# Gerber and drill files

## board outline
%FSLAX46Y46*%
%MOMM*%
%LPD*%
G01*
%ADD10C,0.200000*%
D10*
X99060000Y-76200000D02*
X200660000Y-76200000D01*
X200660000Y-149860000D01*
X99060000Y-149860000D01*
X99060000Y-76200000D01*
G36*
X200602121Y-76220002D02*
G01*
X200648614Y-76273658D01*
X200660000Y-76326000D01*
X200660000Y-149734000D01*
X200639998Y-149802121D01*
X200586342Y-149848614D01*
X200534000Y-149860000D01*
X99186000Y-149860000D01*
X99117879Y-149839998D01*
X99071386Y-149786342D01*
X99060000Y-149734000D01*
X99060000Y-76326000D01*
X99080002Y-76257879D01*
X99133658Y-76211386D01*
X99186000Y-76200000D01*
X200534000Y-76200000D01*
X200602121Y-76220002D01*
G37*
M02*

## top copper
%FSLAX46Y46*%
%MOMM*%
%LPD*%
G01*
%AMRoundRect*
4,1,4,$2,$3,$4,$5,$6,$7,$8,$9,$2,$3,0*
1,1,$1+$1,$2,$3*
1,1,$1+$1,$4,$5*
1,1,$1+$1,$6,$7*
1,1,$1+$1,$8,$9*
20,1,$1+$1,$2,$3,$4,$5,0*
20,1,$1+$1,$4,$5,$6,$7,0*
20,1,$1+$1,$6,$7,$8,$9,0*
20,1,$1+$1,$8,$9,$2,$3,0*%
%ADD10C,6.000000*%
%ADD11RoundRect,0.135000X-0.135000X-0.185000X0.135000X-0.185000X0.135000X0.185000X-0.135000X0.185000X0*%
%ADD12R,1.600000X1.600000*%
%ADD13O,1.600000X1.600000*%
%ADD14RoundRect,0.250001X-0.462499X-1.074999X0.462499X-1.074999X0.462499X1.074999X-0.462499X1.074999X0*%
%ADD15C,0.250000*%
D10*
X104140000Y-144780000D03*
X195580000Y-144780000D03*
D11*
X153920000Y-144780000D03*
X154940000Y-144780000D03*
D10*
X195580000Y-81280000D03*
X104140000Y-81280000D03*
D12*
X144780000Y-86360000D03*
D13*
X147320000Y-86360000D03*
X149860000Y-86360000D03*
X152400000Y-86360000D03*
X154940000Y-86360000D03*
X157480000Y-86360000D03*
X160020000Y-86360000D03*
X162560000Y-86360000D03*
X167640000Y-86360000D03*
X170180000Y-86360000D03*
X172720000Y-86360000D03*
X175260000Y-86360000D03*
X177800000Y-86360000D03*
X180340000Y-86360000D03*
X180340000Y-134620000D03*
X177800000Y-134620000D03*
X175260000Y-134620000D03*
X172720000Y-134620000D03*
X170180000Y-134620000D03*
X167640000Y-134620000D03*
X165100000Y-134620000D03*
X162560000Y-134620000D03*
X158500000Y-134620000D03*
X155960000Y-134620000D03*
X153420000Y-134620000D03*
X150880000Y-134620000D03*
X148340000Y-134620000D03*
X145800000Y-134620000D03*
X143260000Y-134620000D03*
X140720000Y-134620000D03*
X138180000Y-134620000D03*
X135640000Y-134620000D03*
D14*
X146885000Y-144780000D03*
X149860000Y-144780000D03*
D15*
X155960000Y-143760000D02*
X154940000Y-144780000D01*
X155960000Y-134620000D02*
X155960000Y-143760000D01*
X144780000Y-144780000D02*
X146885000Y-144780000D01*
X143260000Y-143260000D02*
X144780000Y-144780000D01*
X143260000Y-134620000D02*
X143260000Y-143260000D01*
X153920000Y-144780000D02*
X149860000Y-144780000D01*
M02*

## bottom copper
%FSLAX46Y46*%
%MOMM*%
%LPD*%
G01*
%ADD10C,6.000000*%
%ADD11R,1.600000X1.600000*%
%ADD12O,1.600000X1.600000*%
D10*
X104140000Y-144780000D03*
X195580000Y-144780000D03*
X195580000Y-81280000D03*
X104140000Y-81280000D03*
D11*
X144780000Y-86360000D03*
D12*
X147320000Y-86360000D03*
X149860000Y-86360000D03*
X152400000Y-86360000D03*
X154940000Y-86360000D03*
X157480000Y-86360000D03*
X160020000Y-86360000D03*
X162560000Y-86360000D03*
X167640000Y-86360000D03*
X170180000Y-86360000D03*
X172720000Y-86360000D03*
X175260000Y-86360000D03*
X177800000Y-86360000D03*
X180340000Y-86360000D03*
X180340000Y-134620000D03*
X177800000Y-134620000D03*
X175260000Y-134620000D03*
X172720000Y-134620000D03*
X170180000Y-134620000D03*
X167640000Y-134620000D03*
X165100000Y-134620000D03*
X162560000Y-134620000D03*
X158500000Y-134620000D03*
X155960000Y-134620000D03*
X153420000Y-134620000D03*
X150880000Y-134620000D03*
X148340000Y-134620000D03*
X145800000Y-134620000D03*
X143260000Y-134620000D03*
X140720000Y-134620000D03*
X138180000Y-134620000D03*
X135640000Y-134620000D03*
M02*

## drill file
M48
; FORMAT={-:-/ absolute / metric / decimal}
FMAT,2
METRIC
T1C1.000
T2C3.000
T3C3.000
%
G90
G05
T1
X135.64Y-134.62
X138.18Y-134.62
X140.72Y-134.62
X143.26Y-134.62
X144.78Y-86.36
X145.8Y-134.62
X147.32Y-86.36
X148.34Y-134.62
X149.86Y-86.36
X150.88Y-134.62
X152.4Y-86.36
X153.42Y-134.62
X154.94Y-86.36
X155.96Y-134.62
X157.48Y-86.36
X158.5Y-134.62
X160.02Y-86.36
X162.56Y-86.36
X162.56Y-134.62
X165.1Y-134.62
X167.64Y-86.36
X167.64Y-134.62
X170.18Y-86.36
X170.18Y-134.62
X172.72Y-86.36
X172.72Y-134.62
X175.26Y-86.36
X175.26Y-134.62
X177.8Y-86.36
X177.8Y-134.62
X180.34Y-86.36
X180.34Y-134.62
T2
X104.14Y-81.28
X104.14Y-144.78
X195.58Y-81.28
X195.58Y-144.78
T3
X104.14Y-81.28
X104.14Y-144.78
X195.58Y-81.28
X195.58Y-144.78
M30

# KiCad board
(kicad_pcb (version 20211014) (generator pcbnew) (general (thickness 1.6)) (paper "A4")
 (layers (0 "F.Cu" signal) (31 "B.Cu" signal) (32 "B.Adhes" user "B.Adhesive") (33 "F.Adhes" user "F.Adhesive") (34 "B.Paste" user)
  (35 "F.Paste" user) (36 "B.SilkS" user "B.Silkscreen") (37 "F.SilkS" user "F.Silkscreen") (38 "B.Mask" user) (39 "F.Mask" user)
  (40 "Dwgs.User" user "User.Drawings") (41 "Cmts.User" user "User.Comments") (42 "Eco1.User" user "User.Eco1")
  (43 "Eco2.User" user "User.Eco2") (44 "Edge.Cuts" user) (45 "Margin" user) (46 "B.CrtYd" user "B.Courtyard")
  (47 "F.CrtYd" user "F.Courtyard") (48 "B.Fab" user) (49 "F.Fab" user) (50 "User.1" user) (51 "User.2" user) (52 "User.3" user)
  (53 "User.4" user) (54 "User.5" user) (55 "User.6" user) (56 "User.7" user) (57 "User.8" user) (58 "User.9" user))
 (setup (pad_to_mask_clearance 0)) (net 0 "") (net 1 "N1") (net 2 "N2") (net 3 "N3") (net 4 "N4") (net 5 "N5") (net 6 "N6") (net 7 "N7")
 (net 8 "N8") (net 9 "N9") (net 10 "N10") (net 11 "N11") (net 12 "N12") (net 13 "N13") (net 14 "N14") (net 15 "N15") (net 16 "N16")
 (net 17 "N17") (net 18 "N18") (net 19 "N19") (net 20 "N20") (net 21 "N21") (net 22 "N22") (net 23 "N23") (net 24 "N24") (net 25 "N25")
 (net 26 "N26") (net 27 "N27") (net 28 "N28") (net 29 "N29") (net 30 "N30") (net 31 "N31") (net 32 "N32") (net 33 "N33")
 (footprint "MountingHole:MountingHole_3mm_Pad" (layer "F.Cu") (at 104.14 144.78)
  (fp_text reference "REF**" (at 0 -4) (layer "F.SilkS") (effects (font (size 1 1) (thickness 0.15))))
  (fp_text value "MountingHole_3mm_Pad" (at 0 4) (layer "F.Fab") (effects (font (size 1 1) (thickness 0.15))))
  (pad "1" thru_hole circle (at 0 0) (size 6 6) (drill 3) (layers *.Cu *.Mask)))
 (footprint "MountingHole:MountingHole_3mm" (layer "F.Cu") (at 195.58 81.28)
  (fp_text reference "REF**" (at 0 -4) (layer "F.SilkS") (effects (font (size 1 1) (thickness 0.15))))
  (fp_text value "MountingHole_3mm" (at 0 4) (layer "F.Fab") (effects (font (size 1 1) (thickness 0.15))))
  (pad "" np_thru_hole circle (at 0 0) (size 3 3) (drill 3) (layers *.Cu *.Mask)))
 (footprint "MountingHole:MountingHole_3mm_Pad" (layer "F.Cu") (at 195.58 144.78)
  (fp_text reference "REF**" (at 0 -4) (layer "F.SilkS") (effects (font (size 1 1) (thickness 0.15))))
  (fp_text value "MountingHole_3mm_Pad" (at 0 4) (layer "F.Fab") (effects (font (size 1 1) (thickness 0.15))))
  (pad "1" thru_hole circle (at 0 0) (size 6 6) (drill 3) (layers *.Cu *.Mask)))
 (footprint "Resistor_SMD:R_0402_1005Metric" (layer "F.Cu") (at 154.43 144.78)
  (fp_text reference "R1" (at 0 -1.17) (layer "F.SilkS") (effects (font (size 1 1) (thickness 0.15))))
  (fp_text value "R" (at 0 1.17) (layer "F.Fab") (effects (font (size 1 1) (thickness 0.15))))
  (pad "1" smd roundrect (at -0.51 0) (size 0.54 0.64) (layers "F.Cu" "F.Paste" "F.Mask") (roundrect_rratio 0.25) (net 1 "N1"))
  (pad "2" smd roundrect (at 0.51 0) (size 0.54 0.64) (layers "F.Cu" "F.Paste" "F.Mask") (roundrect_rratio 0.25) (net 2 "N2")))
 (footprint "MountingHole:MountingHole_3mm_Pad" (layer "F.Cu") (at 195.58 81.28)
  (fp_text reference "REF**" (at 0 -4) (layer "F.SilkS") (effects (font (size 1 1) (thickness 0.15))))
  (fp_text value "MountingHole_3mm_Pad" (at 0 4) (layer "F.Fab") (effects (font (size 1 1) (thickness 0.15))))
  (pad "1" thru_hole circle (at 0 0) (size 6 6) (drill 3) (layers *.Cu *.Mask)))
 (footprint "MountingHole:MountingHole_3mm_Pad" (layer "F.Cu") (at 104.14 81.28)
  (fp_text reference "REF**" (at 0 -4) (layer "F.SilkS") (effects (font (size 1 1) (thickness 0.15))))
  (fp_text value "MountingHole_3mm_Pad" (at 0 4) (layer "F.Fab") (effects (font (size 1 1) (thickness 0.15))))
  (pad "1" thru_hole circle (at 0 0) (size 6 6) (drill 3) (layers *.Cu *.Mask)))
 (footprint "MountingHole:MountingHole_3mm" (layer "F.Cu") (at 104.14 81.28)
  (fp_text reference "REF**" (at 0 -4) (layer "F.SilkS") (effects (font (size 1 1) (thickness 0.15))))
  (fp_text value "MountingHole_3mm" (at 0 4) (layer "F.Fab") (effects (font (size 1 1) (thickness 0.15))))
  (pad "" np_thru_hole circle (at 0 0) (size 3 3) (drill 3) (layers *.Cu *.Mask)))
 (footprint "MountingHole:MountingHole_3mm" (layer "F.Cu") (at 104.14 144.78)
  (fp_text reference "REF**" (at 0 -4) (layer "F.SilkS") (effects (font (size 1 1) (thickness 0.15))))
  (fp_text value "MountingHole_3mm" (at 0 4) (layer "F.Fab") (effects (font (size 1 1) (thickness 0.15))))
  (pad "" np_thru_hole circle (at 0 0) (size 3 3) (drill 3) (layers *.Cu *.Mask)))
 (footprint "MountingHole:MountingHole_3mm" (layer "F.Cu") (at 195.58 144.78)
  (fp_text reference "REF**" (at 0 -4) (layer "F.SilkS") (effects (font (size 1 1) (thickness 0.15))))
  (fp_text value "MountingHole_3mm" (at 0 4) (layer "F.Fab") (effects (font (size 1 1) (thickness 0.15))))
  (pad "" np_thru_hole circle (at 0 0) (size 3 3) (drill 3) (layers *.Cu *.Mask)))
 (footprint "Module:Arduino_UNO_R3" (layer "F.Cu") (at 144.78 86.36)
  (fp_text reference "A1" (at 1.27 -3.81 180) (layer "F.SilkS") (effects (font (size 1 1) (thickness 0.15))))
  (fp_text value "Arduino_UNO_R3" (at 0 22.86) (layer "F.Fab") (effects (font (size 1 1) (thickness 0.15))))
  (pad "1" thru_hole rect (at 0 0 90) (size 1.6 1.6) (drill 1) (layers *.Cu *.Mask) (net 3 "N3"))
  (pad "2" thru_hole oval (at 2.54 0 90) (size 1.6 1.6) (drill 1) (layers *.Cu *.Mask) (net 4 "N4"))
  (pad "3" thru_hole oval (at 5.08 0 90) (size 1.6 1.6) (drill 1) (layers *.Cu *.Mask) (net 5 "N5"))
  (pad "4" thru_hole oval (at 7.62 0 90) (size 1.6 1.6) (drill 1) (layers *.Cu *.Mask) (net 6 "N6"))
  (pad "5" thru_hole oval (at 10.16 0 90) (size 1.6 1.6) (drill 1) (layers *.Cu *.Mask) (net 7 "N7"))
  (pad "6" thru_hole oval (at 12.7 0 90) (size 1.6 1.6) (drill 1) (layers *.Cu *.Mask) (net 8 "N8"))
  (pad "7" thru_hole oval (at 15.24 0 90) (size 1.6 1.6) (drill 1) (layers *.Cu *.Mask) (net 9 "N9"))
  (pad "8" thru_hole oval (at 17.78 0 90) (size 1.6 1.6) (drill 1) (layers *.Cu *.Mask) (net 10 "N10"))
  (pad "9" thru_hole oval (at 22.86 0 90) (size 1.6 1.6) (drill 1) (layers *.Cu *.Mask) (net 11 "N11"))
  (pad "10" thru_hole oval (at 25.4 0 90) (size 1.6 1.6) (drill 1) (layers *.Cu *.Mask) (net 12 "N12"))
  (pad "11" thru_hole oval (at 27.94 0 90) (size 1.6 1.6) (drill 1) (layers *.Cu *.Mask) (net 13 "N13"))
  (pad "12" thru_hole oval (at 30.48 0 90) (size 1.6 1.6) (drill 1) (layers *.Cu *.Mask) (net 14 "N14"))
  (pad "13" thru_hole oval (at 33.02 0 90) (size 1.6 1.6) (drill 1) (layers *.Cu *.Mask) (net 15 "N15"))
  (pad "14" thru_hole oval (at 35.56 0 90) (size 1.6 1.6) (drill 1) (layers *.Cu *.Mask) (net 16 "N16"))
  (pad "15" thru_hole oval (at 35.56 48.26 90) (size 1.6 1.6) (drill 1) (layers *.Cu *.Mask) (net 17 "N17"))
  (pad "16" thru_hole oval (at 33.02 48.26 90) (size 1.6 1.6) (drill 1) (layers *.Cu *.Mask) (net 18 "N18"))
  (pad "17" thru_hole oval (at 30.48 48.26 90) (size 1.6 1.6) (drill 1) (layers *.Cu *.Mask) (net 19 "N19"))
  (pad "18" thru_hole oval (at 27.94 48.26 90) (size 1.6 1.6) (drill 1) (layers *.Cu *.Mask) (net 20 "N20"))
  (pad "19" thru_hole oval (at 25.4 48.26 90) (size 1.6 1.6) (drill 1) (layers *.Cu *.Mask) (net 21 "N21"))
  (pad "20" thru_hole oval (at 22.86 48.26 90) (size 1.6 1.6) (drill 1) (layers *.Cu *.Mask) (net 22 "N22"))
  (pad "21" thru_hole oval (at 20.32 48.26 90) (size 1.6 1.6) (drill 1) (layers *.Cu *.Mask) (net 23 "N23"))
  (pad "22" thru_hole oval (at 17.78 48.26 90) (size 1.6 1.6) (drill 1) (layers *.Cu *.Mask) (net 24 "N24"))
  (pad "23" thru_hole oval (at 13.72 48.26 90) (size 1.6 1.6) (drill 1) (layers *.Cu *.Mask) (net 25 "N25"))
  (pad "24" thru_hole oval (at 11.18 48.26 90) (size 1.6 1.6) (drill 1) (layers *.Cu *.Mask) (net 2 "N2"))
  (pad "25" thru_hole oval (at 8.64 48.26 90) (size 1.6 1.6) (drill 1) (layers *.Cu *.Mask) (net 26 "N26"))
  (pad "26" thru_hole oval (at 6.1 48.26 90) (size 1.6 1.6) (drill 1) (layers *.Cu *.Mask) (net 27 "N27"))
  (pad "27" thru_hole oval (at 3.56 48.26 90) (size 1.6 1.6) (drill 1) (layers *.Cu *.Mask) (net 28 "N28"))
  (pad "28" thru_hole oval (at 1.02 48.26 90) (size 1.6 1.6) (drill 1) (layers *.Cu *.Mask) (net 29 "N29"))
  (pad "29" thru_hole oval (at -1.52 48.26 90) (size 1.6 1.6) (drill 1) (layers *.Cu *.Mask) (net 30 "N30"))
  (pad "30" thru_hole oval (at -4.06 48.26 90) (size 1.6 1.6) (drill 1) (layers *.Cu *.Mask) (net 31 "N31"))
  (pad "31" thru_hole oval (at -6.6 48.26 90) (size 1.6 1.6) (drill 1) (layers *.Cu *.Mask) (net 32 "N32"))
  (pad "32" thru_hole oval (at -9.14 48.26 90) (size 1.6 1.6) (drill 1) (layers *.Cu *.Mask) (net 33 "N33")))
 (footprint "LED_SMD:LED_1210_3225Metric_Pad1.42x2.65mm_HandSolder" (layer "F.Cu") (at 148.3725 144.78)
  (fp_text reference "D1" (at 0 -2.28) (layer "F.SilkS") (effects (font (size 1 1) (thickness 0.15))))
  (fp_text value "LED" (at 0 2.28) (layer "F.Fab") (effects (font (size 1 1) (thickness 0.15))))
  (pad "1" smd roundrect (at -1.4875 0) (size 1.425 2.65) (layers "F.Cu" "F.Paste" "F.Mask") (roundrect_rratio 0.175439) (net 30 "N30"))
  (pad "2" smd roundrect (at 1.4875 0) (size 1.425 2.65) (layers "F.Cu" "F.Paste" "F.Mask") (roundrect_rratio 0.175439) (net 1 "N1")))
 (gr_rect (start 99.06 76.2) (end 200.66 149.86) (layer "Edge.Cuts") (width 0.2) (fill none))
 (segment (start 155.96 143.76) (end 154.94 144.78) (width 0.25) (layer "F.Cu") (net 2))
 (segment (start 155.96 134.62) (end 155.96 143.76) (width 0.25) (layer "F.Cu") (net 2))
 (segment (start 144.78 144.78) (end 146.885 144.78) (width 0.25) (layer "F.Cu") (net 30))
 (segment (start 143.26 143.26) (end 144.78 144.78) (width 0.25) (layer "F.Cu") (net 30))
 (segment (start 143.26 134.62) (end 143.26 143.26) (width 0.25) (layer "F.Cu") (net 30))
 (segment (start 153.92 144.78) (end 149.86 144.78) (width 0.25) (layer "F.Cu") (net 1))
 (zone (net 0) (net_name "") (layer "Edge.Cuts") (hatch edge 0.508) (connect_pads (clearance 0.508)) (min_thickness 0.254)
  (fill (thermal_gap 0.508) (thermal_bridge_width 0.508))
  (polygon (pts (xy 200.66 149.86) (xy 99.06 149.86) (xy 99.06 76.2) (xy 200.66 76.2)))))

